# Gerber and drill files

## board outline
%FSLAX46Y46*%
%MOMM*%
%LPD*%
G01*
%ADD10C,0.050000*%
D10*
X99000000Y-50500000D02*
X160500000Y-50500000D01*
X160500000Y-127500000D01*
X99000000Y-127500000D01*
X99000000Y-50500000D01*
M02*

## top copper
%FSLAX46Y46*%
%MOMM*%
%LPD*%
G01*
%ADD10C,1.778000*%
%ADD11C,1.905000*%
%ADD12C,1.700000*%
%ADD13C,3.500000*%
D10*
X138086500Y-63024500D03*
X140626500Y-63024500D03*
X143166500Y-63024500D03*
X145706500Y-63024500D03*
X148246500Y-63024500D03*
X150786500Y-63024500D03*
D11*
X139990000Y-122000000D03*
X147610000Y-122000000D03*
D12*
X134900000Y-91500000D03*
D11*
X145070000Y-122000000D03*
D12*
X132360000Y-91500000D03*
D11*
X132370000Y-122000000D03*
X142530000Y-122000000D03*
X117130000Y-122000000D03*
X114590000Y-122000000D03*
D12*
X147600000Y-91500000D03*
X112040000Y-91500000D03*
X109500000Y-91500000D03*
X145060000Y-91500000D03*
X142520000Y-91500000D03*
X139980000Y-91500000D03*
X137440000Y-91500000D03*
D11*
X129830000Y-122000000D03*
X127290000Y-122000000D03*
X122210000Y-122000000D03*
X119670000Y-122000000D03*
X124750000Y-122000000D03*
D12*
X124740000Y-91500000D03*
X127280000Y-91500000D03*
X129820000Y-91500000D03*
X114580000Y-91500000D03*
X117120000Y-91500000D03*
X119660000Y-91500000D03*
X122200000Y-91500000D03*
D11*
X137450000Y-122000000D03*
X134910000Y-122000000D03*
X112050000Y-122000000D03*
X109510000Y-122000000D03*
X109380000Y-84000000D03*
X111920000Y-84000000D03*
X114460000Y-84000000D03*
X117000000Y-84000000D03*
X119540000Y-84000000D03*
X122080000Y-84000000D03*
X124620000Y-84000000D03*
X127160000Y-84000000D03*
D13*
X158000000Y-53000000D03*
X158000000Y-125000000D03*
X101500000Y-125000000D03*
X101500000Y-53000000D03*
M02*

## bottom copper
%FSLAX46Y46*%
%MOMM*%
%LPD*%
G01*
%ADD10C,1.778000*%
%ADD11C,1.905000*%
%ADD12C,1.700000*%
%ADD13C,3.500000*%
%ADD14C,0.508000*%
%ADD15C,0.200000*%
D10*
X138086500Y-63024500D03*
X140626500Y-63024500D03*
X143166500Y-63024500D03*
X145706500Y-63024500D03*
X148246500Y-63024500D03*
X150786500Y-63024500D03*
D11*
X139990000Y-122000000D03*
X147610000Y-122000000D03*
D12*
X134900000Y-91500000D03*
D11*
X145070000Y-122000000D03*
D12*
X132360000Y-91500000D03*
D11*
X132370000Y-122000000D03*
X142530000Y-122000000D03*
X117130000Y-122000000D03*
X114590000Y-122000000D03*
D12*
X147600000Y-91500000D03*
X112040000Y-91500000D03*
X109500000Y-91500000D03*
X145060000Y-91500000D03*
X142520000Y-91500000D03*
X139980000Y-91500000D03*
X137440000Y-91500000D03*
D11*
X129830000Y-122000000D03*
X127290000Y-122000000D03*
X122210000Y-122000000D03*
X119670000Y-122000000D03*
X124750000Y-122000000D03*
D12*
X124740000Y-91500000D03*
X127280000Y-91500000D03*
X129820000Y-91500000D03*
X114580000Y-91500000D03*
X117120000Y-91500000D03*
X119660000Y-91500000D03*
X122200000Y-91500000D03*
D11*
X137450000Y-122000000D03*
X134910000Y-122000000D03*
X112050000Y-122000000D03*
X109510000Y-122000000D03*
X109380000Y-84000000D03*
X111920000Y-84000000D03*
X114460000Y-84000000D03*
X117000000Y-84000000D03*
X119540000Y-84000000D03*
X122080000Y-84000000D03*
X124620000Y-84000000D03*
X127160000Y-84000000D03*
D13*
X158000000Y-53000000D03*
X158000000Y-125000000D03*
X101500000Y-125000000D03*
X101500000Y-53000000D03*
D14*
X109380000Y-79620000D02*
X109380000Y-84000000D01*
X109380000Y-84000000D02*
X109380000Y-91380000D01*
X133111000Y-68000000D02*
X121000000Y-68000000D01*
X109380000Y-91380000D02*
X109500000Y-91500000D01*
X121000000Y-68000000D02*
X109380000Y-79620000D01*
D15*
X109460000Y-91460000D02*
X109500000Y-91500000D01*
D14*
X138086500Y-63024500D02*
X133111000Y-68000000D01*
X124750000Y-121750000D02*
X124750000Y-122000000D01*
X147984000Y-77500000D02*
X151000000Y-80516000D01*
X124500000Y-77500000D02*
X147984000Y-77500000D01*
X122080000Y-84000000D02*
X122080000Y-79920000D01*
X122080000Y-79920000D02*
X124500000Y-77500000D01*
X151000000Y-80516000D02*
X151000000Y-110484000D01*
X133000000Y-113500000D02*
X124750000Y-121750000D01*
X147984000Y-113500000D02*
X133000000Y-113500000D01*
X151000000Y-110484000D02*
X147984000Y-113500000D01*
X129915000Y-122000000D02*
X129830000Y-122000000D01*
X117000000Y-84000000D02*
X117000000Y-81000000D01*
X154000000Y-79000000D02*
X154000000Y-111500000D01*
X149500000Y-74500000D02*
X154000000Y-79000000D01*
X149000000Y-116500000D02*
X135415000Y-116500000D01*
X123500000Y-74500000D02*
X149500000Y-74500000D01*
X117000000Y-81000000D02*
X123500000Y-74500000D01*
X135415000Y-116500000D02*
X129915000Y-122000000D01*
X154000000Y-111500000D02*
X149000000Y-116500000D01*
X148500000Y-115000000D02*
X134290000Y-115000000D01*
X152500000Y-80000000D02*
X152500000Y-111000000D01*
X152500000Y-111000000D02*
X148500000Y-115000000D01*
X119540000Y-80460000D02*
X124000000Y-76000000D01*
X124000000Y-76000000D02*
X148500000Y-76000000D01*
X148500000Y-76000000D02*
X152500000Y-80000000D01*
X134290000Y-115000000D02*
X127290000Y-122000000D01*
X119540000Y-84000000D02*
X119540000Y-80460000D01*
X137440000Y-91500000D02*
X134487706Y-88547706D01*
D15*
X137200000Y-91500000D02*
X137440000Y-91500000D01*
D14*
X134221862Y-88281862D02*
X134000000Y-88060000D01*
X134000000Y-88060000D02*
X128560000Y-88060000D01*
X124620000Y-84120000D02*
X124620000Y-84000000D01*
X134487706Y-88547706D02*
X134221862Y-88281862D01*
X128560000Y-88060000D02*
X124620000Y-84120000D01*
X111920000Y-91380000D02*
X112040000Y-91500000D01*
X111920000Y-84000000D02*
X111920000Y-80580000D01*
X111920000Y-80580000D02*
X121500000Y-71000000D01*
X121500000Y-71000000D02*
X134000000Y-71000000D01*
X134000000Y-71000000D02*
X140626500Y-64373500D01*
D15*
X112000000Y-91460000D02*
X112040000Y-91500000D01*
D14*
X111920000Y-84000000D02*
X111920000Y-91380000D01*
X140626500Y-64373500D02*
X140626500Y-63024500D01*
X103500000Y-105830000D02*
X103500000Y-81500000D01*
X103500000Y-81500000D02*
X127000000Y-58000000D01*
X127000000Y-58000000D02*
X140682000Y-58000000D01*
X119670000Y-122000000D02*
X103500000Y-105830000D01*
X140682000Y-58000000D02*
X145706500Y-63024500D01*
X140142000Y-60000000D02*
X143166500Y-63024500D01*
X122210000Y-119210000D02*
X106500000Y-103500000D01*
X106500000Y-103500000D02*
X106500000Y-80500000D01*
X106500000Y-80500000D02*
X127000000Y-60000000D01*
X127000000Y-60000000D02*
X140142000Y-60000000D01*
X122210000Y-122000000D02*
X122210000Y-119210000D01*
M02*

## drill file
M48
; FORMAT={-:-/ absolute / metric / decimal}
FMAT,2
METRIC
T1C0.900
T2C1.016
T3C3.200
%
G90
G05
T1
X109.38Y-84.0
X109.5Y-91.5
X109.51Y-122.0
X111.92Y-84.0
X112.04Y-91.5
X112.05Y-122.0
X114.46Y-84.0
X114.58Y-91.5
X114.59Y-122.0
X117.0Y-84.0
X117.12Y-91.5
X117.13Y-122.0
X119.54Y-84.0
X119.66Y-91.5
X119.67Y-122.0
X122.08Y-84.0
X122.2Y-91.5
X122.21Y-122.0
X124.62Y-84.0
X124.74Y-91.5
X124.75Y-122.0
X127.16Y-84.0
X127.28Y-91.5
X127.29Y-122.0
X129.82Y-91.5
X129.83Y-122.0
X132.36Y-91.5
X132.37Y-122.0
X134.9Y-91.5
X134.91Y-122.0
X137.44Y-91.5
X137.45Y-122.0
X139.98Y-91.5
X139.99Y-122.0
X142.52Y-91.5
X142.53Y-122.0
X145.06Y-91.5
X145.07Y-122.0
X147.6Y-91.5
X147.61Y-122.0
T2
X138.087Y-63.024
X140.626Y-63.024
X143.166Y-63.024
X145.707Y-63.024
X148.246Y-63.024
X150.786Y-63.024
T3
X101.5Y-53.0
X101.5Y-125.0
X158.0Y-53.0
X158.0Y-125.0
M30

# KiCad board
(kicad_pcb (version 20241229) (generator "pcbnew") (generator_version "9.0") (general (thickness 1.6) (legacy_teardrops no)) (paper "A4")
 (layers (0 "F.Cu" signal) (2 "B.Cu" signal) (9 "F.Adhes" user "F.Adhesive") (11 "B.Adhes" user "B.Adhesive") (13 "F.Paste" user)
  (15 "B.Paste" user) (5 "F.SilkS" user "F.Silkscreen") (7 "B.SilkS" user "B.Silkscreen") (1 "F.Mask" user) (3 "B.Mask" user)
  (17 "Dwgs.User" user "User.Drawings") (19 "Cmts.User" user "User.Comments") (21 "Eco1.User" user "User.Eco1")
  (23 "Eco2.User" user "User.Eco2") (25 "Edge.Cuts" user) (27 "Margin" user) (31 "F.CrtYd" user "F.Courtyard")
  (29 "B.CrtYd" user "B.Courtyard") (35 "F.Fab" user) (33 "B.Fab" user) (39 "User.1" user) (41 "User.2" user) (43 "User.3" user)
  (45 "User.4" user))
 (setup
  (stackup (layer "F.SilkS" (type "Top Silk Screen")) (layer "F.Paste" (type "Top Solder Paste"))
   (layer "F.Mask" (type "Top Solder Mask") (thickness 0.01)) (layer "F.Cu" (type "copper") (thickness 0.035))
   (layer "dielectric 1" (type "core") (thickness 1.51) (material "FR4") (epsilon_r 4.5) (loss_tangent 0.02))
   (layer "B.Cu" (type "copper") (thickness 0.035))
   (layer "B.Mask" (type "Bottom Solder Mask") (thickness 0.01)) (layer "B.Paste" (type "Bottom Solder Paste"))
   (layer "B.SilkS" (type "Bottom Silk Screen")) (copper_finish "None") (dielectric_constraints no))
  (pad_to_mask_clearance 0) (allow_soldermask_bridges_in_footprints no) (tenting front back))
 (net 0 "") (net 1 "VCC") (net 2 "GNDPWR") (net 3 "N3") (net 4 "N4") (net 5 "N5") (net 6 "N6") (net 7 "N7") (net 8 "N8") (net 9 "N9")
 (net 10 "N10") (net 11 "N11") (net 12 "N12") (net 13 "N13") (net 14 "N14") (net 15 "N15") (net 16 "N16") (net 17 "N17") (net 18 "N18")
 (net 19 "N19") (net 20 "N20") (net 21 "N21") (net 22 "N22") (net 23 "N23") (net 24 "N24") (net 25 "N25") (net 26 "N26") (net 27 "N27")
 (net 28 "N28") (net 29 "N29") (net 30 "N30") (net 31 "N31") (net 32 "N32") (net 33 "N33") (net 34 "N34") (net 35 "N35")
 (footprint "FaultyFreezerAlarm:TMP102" (layer "F.Cu") (at 136.9435 50.896)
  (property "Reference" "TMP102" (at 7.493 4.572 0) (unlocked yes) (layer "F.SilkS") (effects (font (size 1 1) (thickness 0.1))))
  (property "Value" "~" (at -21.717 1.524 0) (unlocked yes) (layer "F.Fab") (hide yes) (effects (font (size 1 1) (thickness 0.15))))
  (pad "1" thru_hole circle (at 1.143 12.1285) (size 1.778 1.778) (drill 1.016) (layers "*.Cu" "*.Mask") (remove_unused_layers no)
   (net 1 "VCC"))
  (pad "2" thru_hole circle (at 3.683 12.1285) (size 1.778 1.778) (drill 1.016) (layers "*.Cu" "*.Mask") (remove_unused_layers no)
   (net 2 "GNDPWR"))
  (pad "3" thru_hole circle (at 6.223 12.1285) (size 1.778 1.778) (drill 1.016) (layers "*.Cu" "*.Mask") (remove_unused_layers no)
   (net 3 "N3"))
  (pad "4" thru_hole circle (at 8.763 12.1285) (size 1.778 1.778) (drill 1.016) (layers "*.Cu" "*.Mask") (remove_unused_layers no)
   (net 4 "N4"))
  (pad "5" thru_hole circle (at 11.303 12.1285) (size 1.778 1.778) (drill 1.016) (layers "*.Cu" "*.Mask") (remove_unused_layers no)
   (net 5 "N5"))
  (pad "6" thru_hole circle (at 13.843 12.1285) (size 1.778 1.778) (drill 1.016) (layers "*.Cu" "*.Mask") (remove_unused_layers no)
   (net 2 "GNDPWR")))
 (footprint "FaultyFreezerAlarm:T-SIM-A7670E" (layer "F.Cu") (at 173.81 136.75 90)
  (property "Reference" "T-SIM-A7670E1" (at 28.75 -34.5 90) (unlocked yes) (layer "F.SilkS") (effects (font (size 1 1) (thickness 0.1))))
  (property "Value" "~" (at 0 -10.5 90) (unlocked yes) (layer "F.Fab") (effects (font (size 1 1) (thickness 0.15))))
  (pad "0" thru_hole circle (at 14.75 -33.82) (size 1.905 1.905) (drill 0.9) (layers "*.Cu" "*.Mask") (remove_unused_layers no) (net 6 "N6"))
  (pad "01" thru_hole circle (at 14.75 -26.2) (size 1.905 1.905) (drill 0.9) (layers "*.Cu" "*.Mask") (remove_unused_layers no) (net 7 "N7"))
  (pad "02" thru_hole circle (at 45.25 -38.91) (size 1.7 1.7) (drill 0.9) (layers "*.Cu" "*.Mask") (remove_unused_layers no) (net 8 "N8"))
  (pad "03" thru_hole circle (at 14.75 -28.74) (size 1.905 1.905) (drill 0.9) (layers "*.Cu" "*.Mask") (remove_unused_layers no)
   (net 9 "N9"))
  (pad "04" thru_hole circle (at 45.25 -41.45) (size 1.7 1.7) (drill 0.9) (layers "*.Cu" "*.Mask") (remove_unused_layers no) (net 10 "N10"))
  (pad "05" thru_hole circle (at 14.75 -41.44) (size 1.905 1.905) (drill 0.9) (layers "*.Cu" "*.Mask") (remove_unused_layers no)
   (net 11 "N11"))
  (pad "06" thru_hole circle (at 14.75 -31.28) (size 1.905 1.905) (drill 0.9) (layers "*.Cu" "*.Mask") (remove_unused_layers no)
   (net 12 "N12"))
  (pad "07" thru_hole circle (at 14.75 -56.68) (size 1.905 1.905) (drill 0.9) (layers "*.Cu" "*.Mask") (remove_unused_layers no)
   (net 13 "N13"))
  (pad "08" thru_hole circle (at 14.75 -59.22) (size 1.905 1.905) (drill 0.9) (layers "*.Cu" "*.Mask") (remove_unused_layers no)
   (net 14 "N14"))
  (pad "09" thru_hole circle (at 45.25 -26.21) (size 1.7 1.7) (drill 0.9) (layers "*.Cu" "*.Mask") (remove_unused_layers no) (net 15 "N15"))
  (pad "10" thru_hole circle (at 45.25 -61.77) (size 1.7 1.7) (drill 0.9) (layers "*.Cu" "*.Mask") (remove_unused_layers no)
   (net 2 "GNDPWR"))
  (pad "11" thru_hole circle (at 45.25 -64.31) (size 1.7 1.7) (drill 0.9) (layers "*.Cu" "*.Mask") (remove_unused_layers no) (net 1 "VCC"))
  (pad "12" thru_hole circle (at 45.25 -28.75) (size 1.7 1.7) (drill 0.9) (layers "*.Cu" "F.Mask") (remove_unused_layers no) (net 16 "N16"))
  (pad "13" thru_hole circle (at 45.25 -31.29) (size 1.7 1.7) (drill 0.9) (layers "*.Cu" "*.Mask") (remove_unused_layers no) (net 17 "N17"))
  (pad "14" thru_hole circle (at 45.25 -33.83) (size 1.7 1.7) (drill 0.9) (layers "*.Cu" "*.Mask") (remove_unused_layers no) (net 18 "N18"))
  (pad "15" thru_hole circle (at 45.25 -36.37) (size 1.7 1.7) (drill 0.9) (layers "*.Cu" "*.Mask") (remove_unused_layers no) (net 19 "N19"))
  (pad "18" thru_hole circle (at 14.75 -43.98) (size 1.905 1.905) (drill 0.9) (layers "*.Cu" "*.Mask") (remove_unused_layers no)
   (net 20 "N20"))
  (pad "19" thru_hole circle (at 14.75 -46.52) (size 1.905 1.905) (drill 0.9) (layers "*.Cu" "*.Mask") (remove_unused_layers no)
   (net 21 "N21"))
  (pad "21" thru_hole circle (at 14.75 -51.6) (size 1.905 1.905) (drill 0.9) (layers "*.Cu" "*.Mask") (remove_unused_layers no) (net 3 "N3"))
  (pad "22" thru_hole circle (at 14.75 -54.14) (size 1.905 1.905) (drill 0.9) (layers "*.Cu" "*.Mask") (remove_unused_layers no)
   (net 4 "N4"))
  (pad "23" thru_hole circle (at 14.75 -49.06) (size 1.905 1.905) (drill 0.9) (layers "*.Cu" "*.Mask") (remove_unused_layers no)
   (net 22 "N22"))
  (pad "25" thru_hole circle (at 45.25 -49.07) (size 1.7 1.7) (drill 0.9) (layers "*.Cu" "*.Mask" "Dwgs.User") (remove_unused_layers no)
   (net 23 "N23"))
  (pad "26" thru_hole circle (at 45.25 -46.53) (size 1.7 1.7) (drill 0.9) (layers "*.Cu" "*.Mask") (remove_unused_layers no) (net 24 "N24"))
  (pad "27" thru_hole circle (at 45.25 -43.99) (size 1.7 1.7) (drill 0.9) (layers "*.Cu" "*.Mask") (remove_unused_layers no) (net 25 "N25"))
  (pad "32" thru_hole circle (at 45.25 -59.23) (size 1.7 1.7) (drill 0.9) (layers "*.Cu" "*.Mask" "Dwgs.User") (remove_unused_layers no)
   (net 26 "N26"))
  (pad "33" thru_hole circle (at 45.25 -56.69) (size 1.7 1.7) (drill 0.9) (layers "*.Cu" "F.Mask") (remove_unused_layers no) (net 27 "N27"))
  (pad "34" thru_hole circle (at 45.25 -54.15) (size 1.7 1.7) (drill 0.9) (layers "*.Cu" "*.Mask") (remove_unused_layers no) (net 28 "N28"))
  (pad "35" thru_hole circle (at 45.25 -51.61) (size 1.7 1.7) (drill 0.9) (layers "*.Cu" "*.Mask") (remove_unused_layers no) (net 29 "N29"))
  (pad "36" thru_hole circle (at 14.75 -36.36) (size 1.905 1.905) (drill 0.9) (layers "*.Cu" "*.Mask") (remove_unused_layers no)
   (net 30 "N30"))
  (pad "39" thru_hole circle (at 14.75 -38.9) (size 1.905 1.905) (drill 0.9) (layers "*.Cu" "F.Mask") (remove_unused_layers no)
   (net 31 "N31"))
  (pad "RX" thru_hole circle (at 14.75 -61.76) (size 1.905 1.905) (drill 0.9) (layers "*.Cu" "*.Mask" "Dwgs.User") (remove_unused_layers no)
   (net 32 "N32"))
  (pad "TX" thru_hole circle (at 14.75 -64.3) (size 1.905 1.905) (drill 0.9) (layers "*.Cu" "*.Mask") (remove_unused_layers no)
   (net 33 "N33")))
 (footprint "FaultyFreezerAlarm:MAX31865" (layer "F.Cu") (at 118.27 84)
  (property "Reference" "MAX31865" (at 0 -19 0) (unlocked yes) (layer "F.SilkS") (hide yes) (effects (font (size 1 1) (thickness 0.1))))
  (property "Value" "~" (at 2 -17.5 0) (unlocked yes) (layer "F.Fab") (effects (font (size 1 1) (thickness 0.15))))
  (pad "1" thru_hole circle (at -8.89 0) (size 1.905 1.905) (drill 0.9) (layers "*.Cu" "*.Mask") (remove_unused_layers no) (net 1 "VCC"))
  (pad "2" thru_hole circle (at -6.35 0) (size 1.905 1.905) (drill 0.9) (layers "*.Cu" "*.Mask") (remove_unused_layers no) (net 2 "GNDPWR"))
  (pad "3" thru_hole circle (at -3.81 0) (size 1.905 1.905) (drill 0.9) (layers "*.Cu" "*.Mask") (remove_unused_layers no) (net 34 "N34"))
  (pad "4" thru_hole circle (at -1.27 0) (size 1.905 1.905) (drill 0.9) (layers "*.Cu" "*.Mask") (remove_unused_layers no) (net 20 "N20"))
  (pad "5" thru_hole circle (at 1.27 0) (size 1.905 1.905) (drill 0.9) (layers "*.Cu" "*.Mask") (remove_unused_layers no) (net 21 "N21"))
  (pad "6" thru_hole circle (at 3.81 0) (size 1.905 1.905) (drill 0.9) (layers "*.Cu" "*.Mask") (remove_unused_layers no) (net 22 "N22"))
  (pad "7" thru_hole circle (at 6.35 0) (size 1.905 1.905) (drill 0.9) (layers "*.Cu" "*.Mask") (remove_unused_layers no) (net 19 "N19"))
  (pad "8" thru_hole circle (at 8.89 0) (size 1.905 1.905) (drill 0.9) (layers "*.Cu" "*.Mask") (remove_unused_layers no) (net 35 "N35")))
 (gr_rect (start 99 50.5) (end 160.5 127.5) (stroke (width 0.05) (type default)) (fill no) (layer "Edge.Cuts"))
 (via (at 158 53) (size 3.5) (drill 3.2) (layers "F.Cu" "B.Cu") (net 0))
 (via (at 158 125) (size 3.5) (drill 3.2) (layers "F.Cu" "B.Cu") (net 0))
 (via (at 101.5 125) (size 3.5) (drill 3.2) (layers "F.Cu" "B.Cu") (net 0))
 (via (at 101.5 53) (size 3.5) (drill 3.2) (layers "F.Cu" "B.Cu") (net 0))
 (segment (start 109.38 79.62) (end 109.38 84) (width 0.508) (layer "B.Cu") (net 1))
 (segment (start 109.38 84) (end 109.38 91.38) (width 0.508) (layer "B.Cu") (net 1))
 (segment (start 133.111 68) (end 121 68) (width 0.508) (layer "B.Cu") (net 1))
 (segment (start 109.38 91.38) (end 109.5 91.5) (width 0.508) (layer "B.Cu") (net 1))
 (segment (start 121 68) (end 109.38 79.62) (width 0.508) (layer "B.Cu") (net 1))
 (segment (start 109.46 91.46) (end 109.5 91.5) (width 0.2) (layer "B.Cu") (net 1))
 (segment (start 138.0865 63.0245) (end 133.111 68) (width 0.508) (layer "B.Cu") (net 1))
 (segment (start 124.75 121.75) (end 124.75 122) (width 0.508) (layer "B.Cu") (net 22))
 (segment (start 147.984 77.5) (end 151 80.516) (width 0.508) (layer "B.Cu") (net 22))
 (segment (start 124.5 77.5) (end 147.984 77.5) (width 0.508) (layer "B.Cu") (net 22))
 (segment (start 122.08 84) (end 122.08 79.92) (width 0.508) (layer "B.Cu") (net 22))
 (segment (start 122.08 79.92) (end 124.5 77.5) (width 0.508) (layer "B.Cu") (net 22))
 (segment (start 151 80.516) (end 151 110.484) (width 0.508) (layer "B.Cu") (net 22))
 (segment (start 133 113.5) (end 124.75 121.75) (width 0.508) (layer "B.Cu") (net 22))
 (segment (start 147.984 113.5) (end 133 113.5) (width 0.508) (layer "B.Cu") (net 22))
 (segment (start 151 110.484) (end 147.984 113.5) (width 0.508) (layer "B.Cu") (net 22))
 (segment (start 129.915 122) (end 129.83 122) (width 0.508) (layer "B.Cu") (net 20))
 (segment (start 117 84) (end 117 81) (width 0.508) (layer "B.Cu") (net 20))
 (segment (start 154 79) (end 154 111.5) (width 0.508) (layer "B.Cu") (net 20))
 (segment (start 149.5 74.5) (end 154 79) (width 0.508) (layer "B.Cu") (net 20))
 (segment (start 149 116.5) (end 135.415 116.5) (width 0.508) (layer "B.Cu") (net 20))
 (segment (start 123.5 74.5) (end 149.5 74.5) (width 0.508) (layer "B.Cu") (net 20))
 (segment (start 117 81) (end 123.5 74.5) (width 0.508) (layer "B.Cu") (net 20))
 (segment (start 135.415 116.5) (end 129.915 122) (width 0.508) (layer "B.Cu") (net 20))
 (segment (start 154 111.5) (end 149 116.5) (width 0.508) (layer "B.Cu") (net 20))
 (segment (start 148.5 115) (end 134.29 115) (width 0.508) (layer "B.Cu") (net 21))
 (segment (start 152.5 80) (end 152.5 111) (width 0.508) (layer "B.Cu") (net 21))
 (segment (start 152.5 111) (end 148.5 115) (width 0.508) (layer "B.Cu") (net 21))
 (segment (start 119.54 80.46) (end 124 76) (width 0.508) (layer "B.Cu") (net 21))
 (segment (start 124 76) (end 148.5 76) (width 0.508) (layer "B.Cu") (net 21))
 (segment (start 148.5 76) (end 152.5 80) (width 0.508) (layer "B.Cu") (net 21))
 (segment (start 134.29 115) (end 127.29 122) (width 0.508) (layer "B.Cu") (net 21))
 (segment (start 119.54 84) (end 119.54 80.46) (width 0.508) (layer "B.Cu") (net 21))
 (segment (start 137.44 91.5) (end 134.487706 88.547706) (width 0.508) (layer "B.Cu") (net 19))
 (segment (start 137.2 91.5) (end 137.44 91.5) (width 0.2) (layer "B.Cu") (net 19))
 (segment (start 134.221862 88.281862) (end 134 88.06) (width 0.508) (layer "B.Cu") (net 19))
 (segment (start 134 88.06) (end 128.56 88.06) (width 0.508) (layer "B.Cu") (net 19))
 (segment (start 124.62 84.12) (end 124.62 84) (width 0.508) (layer "B.Cu") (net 19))
 (segment (start 134.487706 88.547706) (end 134.221862 88.281862) (width 0.508) (layer "B.Cu") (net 19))
 (segment (start 128.56 88.06) (end 124.62 84.12) (width 0.508) (layer "B.Cu") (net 19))
 (segment (start 111.92 91.38) (end 112.04 91.5) (width 0.508) (layer "B.Cu") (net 2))
 (segment (start 111.92 84) (end 111.92 80.58) (width 0.508) (layer "B.Cu") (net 2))
 (segment (start 111.92 80.58) (end 121.5 71) (width 0.508) (layer "B.Cu") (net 2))
 (segment (start 121.5 71) (end 134 71) (width 0.508) (layer "B.Cu") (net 2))
 (segment (start 134 71) (end 140.6265 64.3735) (width 0.508) (layer "B.Cu") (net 2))
 (segment (start 112 91.46) (end 112.04 91.5) (width 0.2) (layer "B.Cu") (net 2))
 (segment (start 111.92 84) (end 111.92 91.38) (width 0.508) (layer "B.Cu") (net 2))
 (segment (start 140.6265 64.3735) (end 140.6265 63.0245) (width 0.508) (layer "B.Cu") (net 2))
 (segment (start 103.5 105.83) (end 103.5 81.5) (width 0.508) (layer "B.Cu") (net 4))
 (segment (start 103.5 81.5) (end 127 58) (width 0.508) (layer "B.Cu") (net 4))
 (segment (start 127 58) (end 140.682 58) (width 0.508) (layer "B.Cu") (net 4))
 (segment (start 119.67 122) (end 103.5 105.83) (width 0.508) (layer "B.Cu") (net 4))
 (segment (start 140.682 58) (end 145.7065 63.0245) (width 0.508) (layer "B.Cu") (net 4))
 (segment (start 140.142 60) (end 143.1665 63.0245) (width 0.508) (layer "B.Cu") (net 3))
 (segment (start 122.21 119.21) (end 106.5 103.5) (width 0.508) (layer "B.Cu") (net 3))
 (segment (start 106.5 103.5) (end 106.5 80.5) (width 0.508) (layer "B.Cu") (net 3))
 (segment (start 106.5 80.5) (end 127 60) (width 0.508) (layer "B.Cu") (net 3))
 (segment (start 127 60) (end 140.142 60) (width 0.508) (layer "B.Cu") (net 3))
 (segment (start 122.21 122) (end 122.21 119.21) (width 0.508) (layer "B.Cu") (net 3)))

